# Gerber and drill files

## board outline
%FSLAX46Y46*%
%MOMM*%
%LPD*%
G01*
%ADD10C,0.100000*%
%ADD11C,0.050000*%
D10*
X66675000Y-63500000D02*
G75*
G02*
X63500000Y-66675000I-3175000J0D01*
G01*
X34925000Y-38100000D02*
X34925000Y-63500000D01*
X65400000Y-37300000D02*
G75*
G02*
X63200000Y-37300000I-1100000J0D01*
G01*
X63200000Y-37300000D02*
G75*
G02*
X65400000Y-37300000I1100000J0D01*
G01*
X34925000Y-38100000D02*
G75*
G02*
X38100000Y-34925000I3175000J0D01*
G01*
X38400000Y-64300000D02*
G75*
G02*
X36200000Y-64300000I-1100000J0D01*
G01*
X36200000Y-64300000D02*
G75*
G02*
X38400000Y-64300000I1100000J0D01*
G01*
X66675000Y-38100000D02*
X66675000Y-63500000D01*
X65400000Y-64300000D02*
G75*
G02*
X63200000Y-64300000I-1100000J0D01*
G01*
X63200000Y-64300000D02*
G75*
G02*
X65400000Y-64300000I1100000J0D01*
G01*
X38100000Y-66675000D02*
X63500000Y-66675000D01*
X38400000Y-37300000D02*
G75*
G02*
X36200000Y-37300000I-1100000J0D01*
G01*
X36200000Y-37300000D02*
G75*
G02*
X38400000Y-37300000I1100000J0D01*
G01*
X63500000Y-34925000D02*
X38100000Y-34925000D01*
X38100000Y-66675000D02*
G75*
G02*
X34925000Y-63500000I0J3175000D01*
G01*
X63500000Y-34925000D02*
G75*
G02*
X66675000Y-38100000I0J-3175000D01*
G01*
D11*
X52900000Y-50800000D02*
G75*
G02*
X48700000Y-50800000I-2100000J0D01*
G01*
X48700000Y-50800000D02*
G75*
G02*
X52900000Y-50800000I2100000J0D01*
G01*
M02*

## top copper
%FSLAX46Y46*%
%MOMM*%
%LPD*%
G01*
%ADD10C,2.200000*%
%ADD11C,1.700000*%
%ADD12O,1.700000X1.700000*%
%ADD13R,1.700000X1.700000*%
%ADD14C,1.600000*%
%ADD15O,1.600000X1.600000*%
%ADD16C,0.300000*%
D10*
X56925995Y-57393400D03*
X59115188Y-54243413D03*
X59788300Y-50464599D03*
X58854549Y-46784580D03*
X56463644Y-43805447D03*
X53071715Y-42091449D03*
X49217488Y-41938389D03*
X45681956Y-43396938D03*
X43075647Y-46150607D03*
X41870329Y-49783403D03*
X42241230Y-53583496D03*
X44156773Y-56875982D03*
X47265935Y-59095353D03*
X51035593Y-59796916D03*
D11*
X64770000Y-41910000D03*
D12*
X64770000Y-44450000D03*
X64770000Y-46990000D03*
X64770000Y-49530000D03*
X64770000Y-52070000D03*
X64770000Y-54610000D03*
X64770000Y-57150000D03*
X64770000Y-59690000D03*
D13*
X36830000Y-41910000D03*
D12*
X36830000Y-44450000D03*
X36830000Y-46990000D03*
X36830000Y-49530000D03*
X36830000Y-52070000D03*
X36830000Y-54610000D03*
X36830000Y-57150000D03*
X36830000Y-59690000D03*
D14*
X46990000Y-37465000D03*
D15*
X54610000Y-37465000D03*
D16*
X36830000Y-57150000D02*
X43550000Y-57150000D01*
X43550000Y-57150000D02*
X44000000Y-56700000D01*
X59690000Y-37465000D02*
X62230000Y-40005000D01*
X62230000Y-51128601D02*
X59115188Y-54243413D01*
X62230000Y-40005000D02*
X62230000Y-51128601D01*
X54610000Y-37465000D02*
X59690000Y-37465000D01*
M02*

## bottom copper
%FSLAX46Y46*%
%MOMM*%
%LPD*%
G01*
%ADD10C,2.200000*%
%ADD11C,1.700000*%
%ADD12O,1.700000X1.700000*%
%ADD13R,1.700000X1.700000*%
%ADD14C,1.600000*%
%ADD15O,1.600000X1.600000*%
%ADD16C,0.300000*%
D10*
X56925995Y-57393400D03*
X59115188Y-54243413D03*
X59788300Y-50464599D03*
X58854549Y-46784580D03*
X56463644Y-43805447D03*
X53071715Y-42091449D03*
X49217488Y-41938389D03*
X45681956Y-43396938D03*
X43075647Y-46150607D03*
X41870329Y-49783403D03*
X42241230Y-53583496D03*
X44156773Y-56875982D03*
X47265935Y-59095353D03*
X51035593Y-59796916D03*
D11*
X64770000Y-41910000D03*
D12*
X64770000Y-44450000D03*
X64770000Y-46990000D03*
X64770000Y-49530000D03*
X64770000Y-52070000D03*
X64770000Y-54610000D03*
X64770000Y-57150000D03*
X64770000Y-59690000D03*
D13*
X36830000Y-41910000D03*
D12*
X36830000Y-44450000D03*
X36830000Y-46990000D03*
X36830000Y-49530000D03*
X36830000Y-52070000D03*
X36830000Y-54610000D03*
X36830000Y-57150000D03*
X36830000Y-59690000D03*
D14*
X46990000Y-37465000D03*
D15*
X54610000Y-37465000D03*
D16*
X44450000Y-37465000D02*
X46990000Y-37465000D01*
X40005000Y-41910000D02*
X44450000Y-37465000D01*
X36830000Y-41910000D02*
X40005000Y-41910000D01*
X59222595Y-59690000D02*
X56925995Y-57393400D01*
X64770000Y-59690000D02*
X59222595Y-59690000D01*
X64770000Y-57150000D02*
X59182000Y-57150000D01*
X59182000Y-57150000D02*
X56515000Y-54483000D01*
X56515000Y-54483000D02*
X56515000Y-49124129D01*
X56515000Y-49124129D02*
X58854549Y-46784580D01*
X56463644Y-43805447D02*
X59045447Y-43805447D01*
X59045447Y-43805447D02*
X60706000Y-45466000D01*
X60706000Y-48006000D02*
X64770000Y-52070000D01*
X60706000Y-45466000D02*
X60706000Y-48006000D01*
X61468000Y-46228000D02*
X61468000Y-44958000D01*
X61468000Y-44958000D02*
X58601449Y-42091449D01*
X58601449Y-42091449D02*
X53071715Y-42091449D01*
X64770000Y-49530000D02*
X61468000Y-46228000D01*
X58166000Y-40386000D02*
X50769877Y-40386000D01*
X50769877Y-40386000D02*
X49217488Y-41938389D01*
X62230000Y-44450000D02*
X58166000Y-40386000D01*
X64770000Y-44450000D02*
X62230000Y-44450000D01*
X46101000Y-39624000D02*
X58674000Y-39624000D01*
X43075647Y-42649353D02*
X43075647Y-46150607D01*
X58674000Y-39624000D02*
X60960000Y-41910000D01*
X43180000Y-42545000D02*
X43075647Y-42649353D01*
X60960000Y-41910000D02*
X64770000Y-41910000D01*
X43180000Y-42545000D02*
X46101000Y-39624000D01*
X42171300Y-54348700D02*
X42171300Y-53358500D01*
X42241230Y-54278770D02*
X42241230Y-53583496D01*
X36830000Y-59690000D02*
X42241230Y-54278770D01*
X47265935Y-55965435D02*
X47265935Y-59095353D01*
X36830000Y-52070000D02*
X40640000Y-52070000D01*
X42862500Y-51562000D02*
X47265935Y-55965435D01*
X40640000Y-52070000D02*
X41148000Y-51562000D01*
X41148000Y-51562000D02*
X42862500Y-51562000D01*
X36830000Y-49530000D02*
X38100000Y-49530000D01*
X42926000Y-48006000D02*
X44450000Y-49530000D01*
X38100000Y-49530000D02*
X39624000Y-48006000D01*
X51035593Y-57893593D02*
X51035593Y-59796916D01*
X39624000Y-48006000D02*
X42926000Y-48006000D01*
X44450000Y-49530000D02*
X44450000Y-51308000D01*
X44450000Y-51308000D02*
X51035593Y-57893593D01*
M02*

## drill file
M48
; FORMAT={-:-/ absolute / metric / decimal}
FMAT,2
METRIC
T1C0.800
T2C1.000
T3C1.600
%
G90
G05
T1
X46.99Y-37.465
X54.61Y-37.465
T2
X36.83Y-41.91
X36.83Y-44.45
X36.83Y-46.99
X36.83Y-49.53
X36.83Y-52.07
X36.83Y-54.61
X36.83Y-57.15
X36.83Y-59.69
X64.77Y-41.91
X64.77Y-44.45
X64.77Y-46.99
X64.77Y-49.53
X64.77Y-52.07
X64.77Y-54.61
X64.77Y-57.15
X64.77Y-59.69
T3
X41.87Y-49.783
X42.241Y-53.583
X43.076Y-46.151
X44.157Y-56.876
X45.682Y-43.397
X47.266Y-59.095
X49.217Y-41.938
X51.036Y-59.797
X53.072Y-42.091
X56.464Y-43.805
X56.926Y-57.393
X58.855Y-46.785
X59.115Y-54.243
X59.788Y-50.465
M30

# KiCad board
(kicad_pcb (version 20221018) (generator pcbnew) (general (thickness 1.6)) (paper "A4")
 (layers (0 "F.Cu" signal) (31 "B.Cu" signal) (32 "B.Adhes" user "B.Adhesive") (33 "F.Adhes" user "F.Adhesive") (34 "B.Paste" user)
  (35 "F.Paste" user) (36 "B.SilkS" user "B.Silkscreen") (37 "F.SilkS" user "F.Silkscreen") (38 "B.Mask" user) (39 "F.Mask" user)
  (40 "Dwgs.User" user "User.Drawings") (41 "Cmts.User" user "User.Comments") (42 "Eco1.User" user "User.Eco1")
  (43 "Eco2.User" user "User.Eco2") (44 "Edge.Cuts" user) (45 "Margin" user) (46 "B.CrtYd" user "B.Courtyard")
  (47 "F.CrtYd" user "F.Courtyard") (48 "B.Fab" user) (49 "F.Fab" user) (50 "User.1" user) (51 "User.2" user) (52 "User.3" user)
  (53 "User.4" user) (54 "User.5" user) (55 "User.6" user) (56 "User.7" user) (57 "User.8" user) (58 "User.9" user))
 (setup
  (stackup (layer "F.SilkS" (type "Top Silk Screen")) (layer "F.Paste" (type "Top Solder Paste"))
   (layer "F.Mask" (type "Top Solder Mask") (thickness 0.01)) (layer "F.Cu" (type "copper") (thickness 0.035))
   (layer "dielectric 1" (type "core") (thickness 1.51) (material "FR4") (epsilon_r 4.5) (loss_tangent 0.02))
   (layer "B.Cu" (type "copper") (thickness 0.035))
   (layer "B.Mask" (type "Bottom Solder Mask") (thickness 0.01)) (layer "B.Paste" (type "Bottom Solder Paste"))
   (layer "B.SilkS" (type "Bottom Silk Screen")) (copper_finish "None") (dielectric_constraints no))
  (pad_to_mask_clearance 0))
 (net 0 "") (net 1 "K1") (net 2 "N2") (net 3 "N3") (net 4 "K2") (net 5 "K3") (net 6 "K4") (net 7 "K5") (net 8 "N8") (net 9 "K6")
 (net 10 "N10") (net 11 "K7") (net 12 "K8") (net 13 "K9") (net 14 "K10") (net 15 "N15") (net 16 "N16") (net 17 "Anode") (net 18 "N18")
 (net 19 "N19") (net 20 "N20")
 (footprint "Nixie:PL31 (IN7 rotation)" (layer "F.Cu") (at 50.8 50.8)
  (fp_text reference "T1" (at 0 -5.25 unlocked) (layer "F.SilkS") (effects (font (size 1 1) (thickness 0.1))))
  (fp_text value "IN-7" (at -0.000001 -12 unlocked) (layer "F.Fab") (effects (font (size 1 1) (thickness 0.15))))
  (fp_circle (center 0 0) (end 2.1 0) (stroke (width 0.05) (type default)) (fill none) (layer "Edge.Cuts"))
  (pad "1" thru_hole circle (at 6.125995 6.5934 181.5) (size 2.2 2.2) (drill 1.6) (layers "*.Cu" "*.Mask") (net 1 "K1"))
  (pad "2" thru_hole circle (at 8.315188 3.443413 181.5) (size 2.2 2.2) (drill 1.6) (layers "*.Cu" "*.Mask") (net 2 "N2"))
  (pad "3" thru_hole circle (at 8.9883 -0.335401 181.5) (size 2.2 2.2) (drill 1.6) (layers "*.Cu" "*.Mask") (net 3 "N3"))
  (pad "4" thru_hole circle (at 8.054549 -4.01542 181.5) (size 2.2 2.2) (drill 1.6) (layers "*.Cu" "*.Mask") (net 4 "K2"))
  (pad "5" thru_hole circle (at 5.663644 -6.994553 181.5) (size 2.2 2.2) (drill 1.6) (layers "*.Cu" "*.Mask") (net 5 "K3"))
  (pad "6" thru_hole circle (at 2.271715 -8.708551 181.5) (size 2.2 2.2) (drill 1.6) (layers "*.Cu" "*.Mask") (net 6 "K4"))
  (pad "7" thru_hole circle (at -1.582512 -8.861611 181.5) (size 2.2 2.2) (drill 1.6) (layers "*.Cu" "*.Mask") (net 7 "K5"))
  (pad "8" thru_hole circle (at -5.118044 -7.403062 181.5) (size 2.2 2.2) (drill 1.6) (layers "*.Cu" "*.Mask") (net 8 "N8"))
  (pad "9" thru_hole circle (at -7.724353 -4.649393 181.5) (size 2.2 2.2) (drill 1.6) (layers "*.Cu" "*.Mask") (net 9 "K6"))
  (pad "10" thru_hole circle (at -8.929671 -1.016597 181.5) (size 2.2 2.2) (drill 1.6) (layers "*.Cu" "*.Mask") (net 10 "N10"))
  (pad "11" thru_hole circle (at -8.55877 2.783496 181.5) (size 2.2 2.2) (drill 1.6) (layers "*.Cu" "*.Mask") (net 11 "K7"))
  (pad "12" thru_hole circle (at -6.643227 6.075982 181.5) (size 2.2 2.2) (drill 1.6) (layers "*.Cu" "*.Mask") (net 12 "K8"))
  (pad "13" thru_hole circle (at -3.534065 8.295353 181.5) (size 2.2 2.2) (drill 1.6) (layers "*.Cu" "*.Mask") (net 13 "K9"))
  (pad "14" thru_hole circle (at 0.235593 8.996916 181.5) (size 2.2 2.2) (drill 1.6) (layers "*.Cu" "*.Mask") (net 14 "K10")))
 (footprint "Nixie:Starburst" (layer "F.Cu") (at 43 63.25)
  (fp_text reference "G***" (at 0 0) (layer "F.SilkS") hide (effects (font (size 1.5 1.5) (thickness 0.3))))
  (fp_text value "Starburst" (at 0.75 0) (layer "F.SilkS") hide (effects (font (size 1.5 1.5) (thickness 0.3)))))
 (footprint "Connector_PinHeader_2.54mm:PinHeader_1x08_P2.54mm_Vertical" (layer "B.Cu") (at 64.77 41.91 180)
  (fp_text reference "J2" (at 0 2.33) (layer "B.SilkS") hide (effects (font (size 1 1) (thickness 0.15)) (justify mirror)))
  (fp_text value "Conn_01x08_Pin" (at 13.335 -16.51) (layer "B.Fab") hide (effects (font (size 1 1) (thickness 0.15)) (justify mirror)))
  (pad "1" thru_hole circle (at 0 0 180) (size 1.7 1.7) (drill 1) (layers "*.Cu" "*.Mask") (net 9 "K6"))
  (pad "2" thru_hole oval (at 0 -2.54 180) (size 1.7 1.7) (drill 1) (layers "*.Cu" "*.Mask") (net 7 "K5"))
  (pad "3" thru_hole oval (at 0 -5.08 180) (size 1.7 1.7) (drill 1) (layers "*.Cu" "*.Mask") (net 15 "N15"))
  (pad "4" thru_hole oval (at 0 -7.62 180) (size 1.7 1.7) (drill 1) (layers "*.Cu" "*.Mask") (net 6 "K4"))
  (pad "5" thru_hole oval (at 0 -10.16 180) (size 1.7 1.7) (drill 1) (layers "*.Cu" "*.Mask") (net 5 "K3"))
  (pad "6" thru_hole oval (at 0 -12.7 180) (size 1.7 1.7) (drill 1) (layers "*.Cu" "*.Mask") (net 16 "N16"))
  (pad "7" thru_hole oval (at 0 -15.24 180) (size 1.7 1.7) (drill 1) (layers "*.Cu" "*.Mask") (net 4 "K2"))
  (pad "8" thru_hole oval (at 0 -17.78 180) (size 1.7 1.7) (drill 1) (layers "*.Cu" "*.Mask") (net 1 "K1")))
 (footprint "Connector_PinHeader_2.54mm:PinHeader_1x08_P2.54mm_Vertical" (layer "B.Cu") (at 36.83 41.91 180)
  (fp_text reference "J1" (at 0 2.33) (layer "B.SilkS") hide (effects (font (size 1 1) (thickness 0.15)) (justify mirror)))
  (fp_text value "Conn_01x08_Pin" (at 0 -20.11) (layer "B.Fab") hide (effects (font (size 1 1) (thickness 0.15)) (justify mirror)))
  (pad "1" thru_hole rect (at 0 0 180) (size 1.7 1.7) (drill 1) (layers "*.Cu" "*.Mask") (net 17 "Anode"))
  (pad "2" thru_hole oval (at 0 -2.54 180) (size 1.7 1.7) (drill 1) (layers "*.Cu" "*.Mask") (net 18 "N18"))
  (pad "3" thru_hole oval (at 0 -5.08 180) (size 1.7 1.7) (drill 1) (layers "*.Cu" "*.Mask") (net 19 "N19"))
  (pad "4" thru_hole oval (at 0 -7.62 180) (size 1.7 1.7) (drill 1) (layers "*.Cu" "*.Mask") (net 14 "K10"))
  (pad "5" thru_hole oval (at 0 -10.16 180) (size 1.7 1.7) (drill 1) (layers "*.Cu" "*.Mask") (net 13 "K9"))
  (pad "6" thru_hole oval (at 0 -12.7 180) (size 1.7 1.7) (drill 1) (layers "*.Cu" "*.Mask") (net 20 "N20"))
  (pad "7" thru_hole oval (at 0 -15.24 180) (size 1.7 1.7) (drill 1) (layers "*.Cu" "*.Mask") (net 12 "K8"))
  (pad "8" thru_hole oval (at 0 -17.78 180) (size 1.7 1.7) (drill 1) (layers "*.Cu" "*.Mask") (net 11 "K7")))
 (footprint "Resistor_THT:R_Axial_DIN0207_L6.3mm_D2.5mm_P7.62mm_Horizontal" (layer "B.Cu") (at 46.99 37.465)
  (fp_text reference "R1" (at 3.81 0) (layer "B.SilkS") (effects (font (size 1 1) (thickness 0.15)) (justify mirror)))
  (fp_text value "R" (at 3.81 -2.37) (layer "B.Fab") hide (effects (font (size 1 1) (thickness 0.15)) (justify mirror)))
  (pad "1" thru_hole circle (at 0 0) (size 1.6 1.6) (drill 0.8) (layers "*.Cu" "*.Mask") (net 17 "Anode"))
  (pad "2" thru_hole oval (at 7.62 0) (size 1.6 1.6) (drill 0.8) (layers "*.Cu" "*.Mask") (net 2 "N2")))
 (gr_arc (start 66.675 63.5) (mid 65.745064 65.745064) (end 63.5 66.675) (stroke (width 0.1) (type default)) (layer "Edge.Cuts"))
 (gr_line (start 34.925 38.1) (end 34.925 63.5) (stroke (width 0.1) (type default)) (layer "Edge.Cuts"))
 (gr_circle (center 64.3 37.3) (end 65.4 37.3) (stroke (width 0.1) (type default)) (fill none) (layer "Edge.Cuts"))
 (gr_arc (start 34.925 38.1) (mid 35.854936 35.854936) (end 38.1 34.925) (stroke (width 0.1) (type default)) (layer "Edge.Cuts"))
 (gr_circle (center 37.3 64.3) (end 38.4 64.3) (stroke (width 0.1) (type default)) (fill none) (layer "Edge.Cuts"))
 (gr_line (start 66.675 38.1) (end 66.675 63.5) (stroke (width 0.1) (type default)) (layer "Edge.Cuts"))
 (gr_circle (center 64.3 64.3) (end 65.4 64.3) (stroke (width 0.1) (type default)) (fill none) (layer "Edge.Cuts"))
 (gr_line (start 38.1 66.675) (end 63.5 66.675) (stroke (width 0.1) (type default)) (layer "Edge.Cuts"))
 (gr_circle (center 37.3 37.3) (end 38.4 37.3) (stroke (width 0.1) (type default)) (fill none) (layer "Edge.Cuts"))
 (gr_line (start 63.5 34.925) (end 38.1 34.925) (stroke (width 0.1) (type default)) (layer "Edge.Cuts"))
 (gr_arc (start 38.1 66.675) (mid 35.854936 65.745064) (end 34.925 63.5) (stroke (width 0.1) (type default)) (layer "Edge.Cuts"))
 (gr_arc (start 63.5 34.925) (mid 65.745064 35.854936) (end 66.675 38.1) (stroke (width 0.1) (type default)) (layer "Edge.Cuts"))
 (segment (start 44.45 37.465) (end 46.99 37.465) (width 0.3) (layer "B.Cu") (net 17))
 (segment (start 40.005 41.91) (end 44.45 37.465) (width 0.3) (layer "B.Cu") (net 17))
 (segment (start 36.83 41.91) (end 40.005 41.91) (width 0.3) (layer "B.Cu") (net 17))
 (segment (start 59.222595 59.69) (end 56.925995 57.3934) (width 0.3) (layer "B.Cu") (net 1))
 (segment (start 64.77 59.69) (end 59.222595 59.69) (width 0.3) (layer "B.Cu") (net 1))
 (segment (start 64.77 57.15) (end 59.182 57.15) (width 0.3) (layer "B.Cu") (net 4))
 (segment (start 59.182 57.15) (end 56.515 54.483) (width 0.3) (layer "B.Cu") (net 4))
 (segment (start 56.515 54.483) (end 56.515 49.124129) (width 0.3) (layer "B.Cu") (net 4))
 (segment (start 56.515 49.124129) (end 58.854549 46.78458) (width 0.3) (layer "B.Cu") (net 4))
 (segment (start 56.463644 43.805447) (end 59.045447 43.805447) (width 0.3) (layer "B.Cu") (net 5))
 (segment (start 59.045447 43.805447) (end 60.706 45.466) (width 0.3) (layer "B.Cu") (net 5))
 (segment (start 60.706 48.006) (end 64.77 52.07) (width 0.3) (layer "B.Cu") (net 5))
 (segment (start 60.706 45.466) (end 60.706 48.006) (width 0.3) (layer "B.Cu") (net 5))
 (segment (start 61.468 46.228) (end 61.468 44.958) (width 0.3) (layer "B.Cu") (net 6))
 (segment (start 61.468 44.958) (end 58.601449 42.091449) (width 0.3) (layer "B.Cu") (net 6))
 (segment (start 58.601449 42.091449) (end 53.071715 42.091449) (width 0.3) (layer "B.Cu") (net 6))
 (segment (start 64.77 49.53) (end 61.468 46.228) (width 0.3) (layer "B.Cu") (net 6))
 (segment (start 58.166 40.386) (end 50.769877 40.386) (width 0.3) (layer "B.Cu") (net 7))
 (segment (start 50.769877 40.386) (end 49.217488 41.938389) (width 0.3) (layer "B.Cu") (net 7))
 (segment (start 62.23 44.45) (end 58.166 40.386) (width 0.3) (layer "B.Cu") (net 7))
 (segment (start 64.77 44.45) (end 62.23 44.45) (width 0.3) (layer "B.Cu") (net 7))
 (segment (start 46.101 39.624) (end 58.674 39.624) (width 0.3) (layer "B.Cu") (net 9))
 (segment (start 43.075647 42.649353) (end 43.075647 46.150607) (width 0.3) (layer "B.Cu") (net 9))
 (segment (start 58.674 39.624) (end 60.96 41.91) (width 0.3) (layer "B.Cu") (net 9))
 (segment (start 43.18 42.545) (end 43.075647 42.649353) (width 0.3) (layer "B.Cu") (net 9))
 (segment (start 60.96 41.91) (end 64.77 41.91) (width 0.3) (layer "B.Cu") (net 9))
 (segment (start 43.18 42.545) (end 46.101 39.624) (width 0.3) (layer "B.Cu") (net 9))
 (segment (start 42.1713 54.3487) (end 42.1713 53.3585) (width 0.3) (layer "B.Cu") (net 11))
 (segment (start 42.24123 54.27877) (end 42.24123 53.583496) (width 0.3) (layer "B.Cu") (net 11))
 (segment (start 36.83 59.69) (end 42.24123 54.27877) (width 0.3) (layer "B.Cu") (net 11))
 (segment (start 36.83 57.15) (end 43.55 57.15) (width 0.3) (layer "F.Cu") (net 12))
 (segment (start 43.55 57.15) (end 44 56.7) (width 0.3) (layer "F.Cu") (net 12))
 (segment (start 47.265935 55.965435) (end 47.265935 59.095353) (width 0.3) (layer "B.Cu") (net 13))
 (segment (start 36.83 52.07) (end 40.64 52.07) (width 0.3) (layer "B.Cu") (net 13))
 (segment (start 42.8625 51.562) (end 47.265935 55.965435) (width 0.3) (layer "B.Cu") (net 13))
 (segment (start 40.64 52.07) (end 41.148 51.562) (width 0.3) (layer "B.Cu") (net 13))
 (segment (start 41.148 51.562) (end 42.8625 51.562) (width 0.3) (layer "B.Cu") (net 13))
 (segment (start 36.83 49.53) (end 38.1 49.53) (width 0.3) (layer "B.Cu") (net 14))
 (segment (start 42.926 48.006) (end 44.45 49.53) (width 0.3) (layer "B.Cu") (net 14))
 (segment (start 38.1 49.53) (end 39.624 48.006) (width 0.3) (layer "B.Cu") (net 14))
 (segment (start 51.035593 57.893593) (end 51.035593 59.796916) (width 0.3) (layer "B.Cu") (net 14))
 (segment (start 39.624 48.006) (end 42.926 48.006) (width 0.3) (layer "B.Cu") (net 14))
 (segment (start 44.45 49.53) (end 44.45 51.308) (width 0.3) (layer "B.Cu") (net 14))
 (segment (start 44.45 51.308) (end 51.035593 57.893593) (width 0.3) (layer "B.Cu") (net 14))
 (segment (start 59.69 37.465) (end 62.23 40.005) (width 0.3) (layer "F.Cu") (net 2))
 (segment (start 62.23 51.128601) (end 59.115188 54.243413) (width 0.3) (layer "F.Cu") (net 2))
 (segment (start 62.23 40.005) (end 62.23 51.128601) (width 0.3) (layer "F.Cu") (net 2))
 (segment (start 54.61 37.465) (end 59.69 37.465) (width 0.3) (layer "F.Cu") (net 2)))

